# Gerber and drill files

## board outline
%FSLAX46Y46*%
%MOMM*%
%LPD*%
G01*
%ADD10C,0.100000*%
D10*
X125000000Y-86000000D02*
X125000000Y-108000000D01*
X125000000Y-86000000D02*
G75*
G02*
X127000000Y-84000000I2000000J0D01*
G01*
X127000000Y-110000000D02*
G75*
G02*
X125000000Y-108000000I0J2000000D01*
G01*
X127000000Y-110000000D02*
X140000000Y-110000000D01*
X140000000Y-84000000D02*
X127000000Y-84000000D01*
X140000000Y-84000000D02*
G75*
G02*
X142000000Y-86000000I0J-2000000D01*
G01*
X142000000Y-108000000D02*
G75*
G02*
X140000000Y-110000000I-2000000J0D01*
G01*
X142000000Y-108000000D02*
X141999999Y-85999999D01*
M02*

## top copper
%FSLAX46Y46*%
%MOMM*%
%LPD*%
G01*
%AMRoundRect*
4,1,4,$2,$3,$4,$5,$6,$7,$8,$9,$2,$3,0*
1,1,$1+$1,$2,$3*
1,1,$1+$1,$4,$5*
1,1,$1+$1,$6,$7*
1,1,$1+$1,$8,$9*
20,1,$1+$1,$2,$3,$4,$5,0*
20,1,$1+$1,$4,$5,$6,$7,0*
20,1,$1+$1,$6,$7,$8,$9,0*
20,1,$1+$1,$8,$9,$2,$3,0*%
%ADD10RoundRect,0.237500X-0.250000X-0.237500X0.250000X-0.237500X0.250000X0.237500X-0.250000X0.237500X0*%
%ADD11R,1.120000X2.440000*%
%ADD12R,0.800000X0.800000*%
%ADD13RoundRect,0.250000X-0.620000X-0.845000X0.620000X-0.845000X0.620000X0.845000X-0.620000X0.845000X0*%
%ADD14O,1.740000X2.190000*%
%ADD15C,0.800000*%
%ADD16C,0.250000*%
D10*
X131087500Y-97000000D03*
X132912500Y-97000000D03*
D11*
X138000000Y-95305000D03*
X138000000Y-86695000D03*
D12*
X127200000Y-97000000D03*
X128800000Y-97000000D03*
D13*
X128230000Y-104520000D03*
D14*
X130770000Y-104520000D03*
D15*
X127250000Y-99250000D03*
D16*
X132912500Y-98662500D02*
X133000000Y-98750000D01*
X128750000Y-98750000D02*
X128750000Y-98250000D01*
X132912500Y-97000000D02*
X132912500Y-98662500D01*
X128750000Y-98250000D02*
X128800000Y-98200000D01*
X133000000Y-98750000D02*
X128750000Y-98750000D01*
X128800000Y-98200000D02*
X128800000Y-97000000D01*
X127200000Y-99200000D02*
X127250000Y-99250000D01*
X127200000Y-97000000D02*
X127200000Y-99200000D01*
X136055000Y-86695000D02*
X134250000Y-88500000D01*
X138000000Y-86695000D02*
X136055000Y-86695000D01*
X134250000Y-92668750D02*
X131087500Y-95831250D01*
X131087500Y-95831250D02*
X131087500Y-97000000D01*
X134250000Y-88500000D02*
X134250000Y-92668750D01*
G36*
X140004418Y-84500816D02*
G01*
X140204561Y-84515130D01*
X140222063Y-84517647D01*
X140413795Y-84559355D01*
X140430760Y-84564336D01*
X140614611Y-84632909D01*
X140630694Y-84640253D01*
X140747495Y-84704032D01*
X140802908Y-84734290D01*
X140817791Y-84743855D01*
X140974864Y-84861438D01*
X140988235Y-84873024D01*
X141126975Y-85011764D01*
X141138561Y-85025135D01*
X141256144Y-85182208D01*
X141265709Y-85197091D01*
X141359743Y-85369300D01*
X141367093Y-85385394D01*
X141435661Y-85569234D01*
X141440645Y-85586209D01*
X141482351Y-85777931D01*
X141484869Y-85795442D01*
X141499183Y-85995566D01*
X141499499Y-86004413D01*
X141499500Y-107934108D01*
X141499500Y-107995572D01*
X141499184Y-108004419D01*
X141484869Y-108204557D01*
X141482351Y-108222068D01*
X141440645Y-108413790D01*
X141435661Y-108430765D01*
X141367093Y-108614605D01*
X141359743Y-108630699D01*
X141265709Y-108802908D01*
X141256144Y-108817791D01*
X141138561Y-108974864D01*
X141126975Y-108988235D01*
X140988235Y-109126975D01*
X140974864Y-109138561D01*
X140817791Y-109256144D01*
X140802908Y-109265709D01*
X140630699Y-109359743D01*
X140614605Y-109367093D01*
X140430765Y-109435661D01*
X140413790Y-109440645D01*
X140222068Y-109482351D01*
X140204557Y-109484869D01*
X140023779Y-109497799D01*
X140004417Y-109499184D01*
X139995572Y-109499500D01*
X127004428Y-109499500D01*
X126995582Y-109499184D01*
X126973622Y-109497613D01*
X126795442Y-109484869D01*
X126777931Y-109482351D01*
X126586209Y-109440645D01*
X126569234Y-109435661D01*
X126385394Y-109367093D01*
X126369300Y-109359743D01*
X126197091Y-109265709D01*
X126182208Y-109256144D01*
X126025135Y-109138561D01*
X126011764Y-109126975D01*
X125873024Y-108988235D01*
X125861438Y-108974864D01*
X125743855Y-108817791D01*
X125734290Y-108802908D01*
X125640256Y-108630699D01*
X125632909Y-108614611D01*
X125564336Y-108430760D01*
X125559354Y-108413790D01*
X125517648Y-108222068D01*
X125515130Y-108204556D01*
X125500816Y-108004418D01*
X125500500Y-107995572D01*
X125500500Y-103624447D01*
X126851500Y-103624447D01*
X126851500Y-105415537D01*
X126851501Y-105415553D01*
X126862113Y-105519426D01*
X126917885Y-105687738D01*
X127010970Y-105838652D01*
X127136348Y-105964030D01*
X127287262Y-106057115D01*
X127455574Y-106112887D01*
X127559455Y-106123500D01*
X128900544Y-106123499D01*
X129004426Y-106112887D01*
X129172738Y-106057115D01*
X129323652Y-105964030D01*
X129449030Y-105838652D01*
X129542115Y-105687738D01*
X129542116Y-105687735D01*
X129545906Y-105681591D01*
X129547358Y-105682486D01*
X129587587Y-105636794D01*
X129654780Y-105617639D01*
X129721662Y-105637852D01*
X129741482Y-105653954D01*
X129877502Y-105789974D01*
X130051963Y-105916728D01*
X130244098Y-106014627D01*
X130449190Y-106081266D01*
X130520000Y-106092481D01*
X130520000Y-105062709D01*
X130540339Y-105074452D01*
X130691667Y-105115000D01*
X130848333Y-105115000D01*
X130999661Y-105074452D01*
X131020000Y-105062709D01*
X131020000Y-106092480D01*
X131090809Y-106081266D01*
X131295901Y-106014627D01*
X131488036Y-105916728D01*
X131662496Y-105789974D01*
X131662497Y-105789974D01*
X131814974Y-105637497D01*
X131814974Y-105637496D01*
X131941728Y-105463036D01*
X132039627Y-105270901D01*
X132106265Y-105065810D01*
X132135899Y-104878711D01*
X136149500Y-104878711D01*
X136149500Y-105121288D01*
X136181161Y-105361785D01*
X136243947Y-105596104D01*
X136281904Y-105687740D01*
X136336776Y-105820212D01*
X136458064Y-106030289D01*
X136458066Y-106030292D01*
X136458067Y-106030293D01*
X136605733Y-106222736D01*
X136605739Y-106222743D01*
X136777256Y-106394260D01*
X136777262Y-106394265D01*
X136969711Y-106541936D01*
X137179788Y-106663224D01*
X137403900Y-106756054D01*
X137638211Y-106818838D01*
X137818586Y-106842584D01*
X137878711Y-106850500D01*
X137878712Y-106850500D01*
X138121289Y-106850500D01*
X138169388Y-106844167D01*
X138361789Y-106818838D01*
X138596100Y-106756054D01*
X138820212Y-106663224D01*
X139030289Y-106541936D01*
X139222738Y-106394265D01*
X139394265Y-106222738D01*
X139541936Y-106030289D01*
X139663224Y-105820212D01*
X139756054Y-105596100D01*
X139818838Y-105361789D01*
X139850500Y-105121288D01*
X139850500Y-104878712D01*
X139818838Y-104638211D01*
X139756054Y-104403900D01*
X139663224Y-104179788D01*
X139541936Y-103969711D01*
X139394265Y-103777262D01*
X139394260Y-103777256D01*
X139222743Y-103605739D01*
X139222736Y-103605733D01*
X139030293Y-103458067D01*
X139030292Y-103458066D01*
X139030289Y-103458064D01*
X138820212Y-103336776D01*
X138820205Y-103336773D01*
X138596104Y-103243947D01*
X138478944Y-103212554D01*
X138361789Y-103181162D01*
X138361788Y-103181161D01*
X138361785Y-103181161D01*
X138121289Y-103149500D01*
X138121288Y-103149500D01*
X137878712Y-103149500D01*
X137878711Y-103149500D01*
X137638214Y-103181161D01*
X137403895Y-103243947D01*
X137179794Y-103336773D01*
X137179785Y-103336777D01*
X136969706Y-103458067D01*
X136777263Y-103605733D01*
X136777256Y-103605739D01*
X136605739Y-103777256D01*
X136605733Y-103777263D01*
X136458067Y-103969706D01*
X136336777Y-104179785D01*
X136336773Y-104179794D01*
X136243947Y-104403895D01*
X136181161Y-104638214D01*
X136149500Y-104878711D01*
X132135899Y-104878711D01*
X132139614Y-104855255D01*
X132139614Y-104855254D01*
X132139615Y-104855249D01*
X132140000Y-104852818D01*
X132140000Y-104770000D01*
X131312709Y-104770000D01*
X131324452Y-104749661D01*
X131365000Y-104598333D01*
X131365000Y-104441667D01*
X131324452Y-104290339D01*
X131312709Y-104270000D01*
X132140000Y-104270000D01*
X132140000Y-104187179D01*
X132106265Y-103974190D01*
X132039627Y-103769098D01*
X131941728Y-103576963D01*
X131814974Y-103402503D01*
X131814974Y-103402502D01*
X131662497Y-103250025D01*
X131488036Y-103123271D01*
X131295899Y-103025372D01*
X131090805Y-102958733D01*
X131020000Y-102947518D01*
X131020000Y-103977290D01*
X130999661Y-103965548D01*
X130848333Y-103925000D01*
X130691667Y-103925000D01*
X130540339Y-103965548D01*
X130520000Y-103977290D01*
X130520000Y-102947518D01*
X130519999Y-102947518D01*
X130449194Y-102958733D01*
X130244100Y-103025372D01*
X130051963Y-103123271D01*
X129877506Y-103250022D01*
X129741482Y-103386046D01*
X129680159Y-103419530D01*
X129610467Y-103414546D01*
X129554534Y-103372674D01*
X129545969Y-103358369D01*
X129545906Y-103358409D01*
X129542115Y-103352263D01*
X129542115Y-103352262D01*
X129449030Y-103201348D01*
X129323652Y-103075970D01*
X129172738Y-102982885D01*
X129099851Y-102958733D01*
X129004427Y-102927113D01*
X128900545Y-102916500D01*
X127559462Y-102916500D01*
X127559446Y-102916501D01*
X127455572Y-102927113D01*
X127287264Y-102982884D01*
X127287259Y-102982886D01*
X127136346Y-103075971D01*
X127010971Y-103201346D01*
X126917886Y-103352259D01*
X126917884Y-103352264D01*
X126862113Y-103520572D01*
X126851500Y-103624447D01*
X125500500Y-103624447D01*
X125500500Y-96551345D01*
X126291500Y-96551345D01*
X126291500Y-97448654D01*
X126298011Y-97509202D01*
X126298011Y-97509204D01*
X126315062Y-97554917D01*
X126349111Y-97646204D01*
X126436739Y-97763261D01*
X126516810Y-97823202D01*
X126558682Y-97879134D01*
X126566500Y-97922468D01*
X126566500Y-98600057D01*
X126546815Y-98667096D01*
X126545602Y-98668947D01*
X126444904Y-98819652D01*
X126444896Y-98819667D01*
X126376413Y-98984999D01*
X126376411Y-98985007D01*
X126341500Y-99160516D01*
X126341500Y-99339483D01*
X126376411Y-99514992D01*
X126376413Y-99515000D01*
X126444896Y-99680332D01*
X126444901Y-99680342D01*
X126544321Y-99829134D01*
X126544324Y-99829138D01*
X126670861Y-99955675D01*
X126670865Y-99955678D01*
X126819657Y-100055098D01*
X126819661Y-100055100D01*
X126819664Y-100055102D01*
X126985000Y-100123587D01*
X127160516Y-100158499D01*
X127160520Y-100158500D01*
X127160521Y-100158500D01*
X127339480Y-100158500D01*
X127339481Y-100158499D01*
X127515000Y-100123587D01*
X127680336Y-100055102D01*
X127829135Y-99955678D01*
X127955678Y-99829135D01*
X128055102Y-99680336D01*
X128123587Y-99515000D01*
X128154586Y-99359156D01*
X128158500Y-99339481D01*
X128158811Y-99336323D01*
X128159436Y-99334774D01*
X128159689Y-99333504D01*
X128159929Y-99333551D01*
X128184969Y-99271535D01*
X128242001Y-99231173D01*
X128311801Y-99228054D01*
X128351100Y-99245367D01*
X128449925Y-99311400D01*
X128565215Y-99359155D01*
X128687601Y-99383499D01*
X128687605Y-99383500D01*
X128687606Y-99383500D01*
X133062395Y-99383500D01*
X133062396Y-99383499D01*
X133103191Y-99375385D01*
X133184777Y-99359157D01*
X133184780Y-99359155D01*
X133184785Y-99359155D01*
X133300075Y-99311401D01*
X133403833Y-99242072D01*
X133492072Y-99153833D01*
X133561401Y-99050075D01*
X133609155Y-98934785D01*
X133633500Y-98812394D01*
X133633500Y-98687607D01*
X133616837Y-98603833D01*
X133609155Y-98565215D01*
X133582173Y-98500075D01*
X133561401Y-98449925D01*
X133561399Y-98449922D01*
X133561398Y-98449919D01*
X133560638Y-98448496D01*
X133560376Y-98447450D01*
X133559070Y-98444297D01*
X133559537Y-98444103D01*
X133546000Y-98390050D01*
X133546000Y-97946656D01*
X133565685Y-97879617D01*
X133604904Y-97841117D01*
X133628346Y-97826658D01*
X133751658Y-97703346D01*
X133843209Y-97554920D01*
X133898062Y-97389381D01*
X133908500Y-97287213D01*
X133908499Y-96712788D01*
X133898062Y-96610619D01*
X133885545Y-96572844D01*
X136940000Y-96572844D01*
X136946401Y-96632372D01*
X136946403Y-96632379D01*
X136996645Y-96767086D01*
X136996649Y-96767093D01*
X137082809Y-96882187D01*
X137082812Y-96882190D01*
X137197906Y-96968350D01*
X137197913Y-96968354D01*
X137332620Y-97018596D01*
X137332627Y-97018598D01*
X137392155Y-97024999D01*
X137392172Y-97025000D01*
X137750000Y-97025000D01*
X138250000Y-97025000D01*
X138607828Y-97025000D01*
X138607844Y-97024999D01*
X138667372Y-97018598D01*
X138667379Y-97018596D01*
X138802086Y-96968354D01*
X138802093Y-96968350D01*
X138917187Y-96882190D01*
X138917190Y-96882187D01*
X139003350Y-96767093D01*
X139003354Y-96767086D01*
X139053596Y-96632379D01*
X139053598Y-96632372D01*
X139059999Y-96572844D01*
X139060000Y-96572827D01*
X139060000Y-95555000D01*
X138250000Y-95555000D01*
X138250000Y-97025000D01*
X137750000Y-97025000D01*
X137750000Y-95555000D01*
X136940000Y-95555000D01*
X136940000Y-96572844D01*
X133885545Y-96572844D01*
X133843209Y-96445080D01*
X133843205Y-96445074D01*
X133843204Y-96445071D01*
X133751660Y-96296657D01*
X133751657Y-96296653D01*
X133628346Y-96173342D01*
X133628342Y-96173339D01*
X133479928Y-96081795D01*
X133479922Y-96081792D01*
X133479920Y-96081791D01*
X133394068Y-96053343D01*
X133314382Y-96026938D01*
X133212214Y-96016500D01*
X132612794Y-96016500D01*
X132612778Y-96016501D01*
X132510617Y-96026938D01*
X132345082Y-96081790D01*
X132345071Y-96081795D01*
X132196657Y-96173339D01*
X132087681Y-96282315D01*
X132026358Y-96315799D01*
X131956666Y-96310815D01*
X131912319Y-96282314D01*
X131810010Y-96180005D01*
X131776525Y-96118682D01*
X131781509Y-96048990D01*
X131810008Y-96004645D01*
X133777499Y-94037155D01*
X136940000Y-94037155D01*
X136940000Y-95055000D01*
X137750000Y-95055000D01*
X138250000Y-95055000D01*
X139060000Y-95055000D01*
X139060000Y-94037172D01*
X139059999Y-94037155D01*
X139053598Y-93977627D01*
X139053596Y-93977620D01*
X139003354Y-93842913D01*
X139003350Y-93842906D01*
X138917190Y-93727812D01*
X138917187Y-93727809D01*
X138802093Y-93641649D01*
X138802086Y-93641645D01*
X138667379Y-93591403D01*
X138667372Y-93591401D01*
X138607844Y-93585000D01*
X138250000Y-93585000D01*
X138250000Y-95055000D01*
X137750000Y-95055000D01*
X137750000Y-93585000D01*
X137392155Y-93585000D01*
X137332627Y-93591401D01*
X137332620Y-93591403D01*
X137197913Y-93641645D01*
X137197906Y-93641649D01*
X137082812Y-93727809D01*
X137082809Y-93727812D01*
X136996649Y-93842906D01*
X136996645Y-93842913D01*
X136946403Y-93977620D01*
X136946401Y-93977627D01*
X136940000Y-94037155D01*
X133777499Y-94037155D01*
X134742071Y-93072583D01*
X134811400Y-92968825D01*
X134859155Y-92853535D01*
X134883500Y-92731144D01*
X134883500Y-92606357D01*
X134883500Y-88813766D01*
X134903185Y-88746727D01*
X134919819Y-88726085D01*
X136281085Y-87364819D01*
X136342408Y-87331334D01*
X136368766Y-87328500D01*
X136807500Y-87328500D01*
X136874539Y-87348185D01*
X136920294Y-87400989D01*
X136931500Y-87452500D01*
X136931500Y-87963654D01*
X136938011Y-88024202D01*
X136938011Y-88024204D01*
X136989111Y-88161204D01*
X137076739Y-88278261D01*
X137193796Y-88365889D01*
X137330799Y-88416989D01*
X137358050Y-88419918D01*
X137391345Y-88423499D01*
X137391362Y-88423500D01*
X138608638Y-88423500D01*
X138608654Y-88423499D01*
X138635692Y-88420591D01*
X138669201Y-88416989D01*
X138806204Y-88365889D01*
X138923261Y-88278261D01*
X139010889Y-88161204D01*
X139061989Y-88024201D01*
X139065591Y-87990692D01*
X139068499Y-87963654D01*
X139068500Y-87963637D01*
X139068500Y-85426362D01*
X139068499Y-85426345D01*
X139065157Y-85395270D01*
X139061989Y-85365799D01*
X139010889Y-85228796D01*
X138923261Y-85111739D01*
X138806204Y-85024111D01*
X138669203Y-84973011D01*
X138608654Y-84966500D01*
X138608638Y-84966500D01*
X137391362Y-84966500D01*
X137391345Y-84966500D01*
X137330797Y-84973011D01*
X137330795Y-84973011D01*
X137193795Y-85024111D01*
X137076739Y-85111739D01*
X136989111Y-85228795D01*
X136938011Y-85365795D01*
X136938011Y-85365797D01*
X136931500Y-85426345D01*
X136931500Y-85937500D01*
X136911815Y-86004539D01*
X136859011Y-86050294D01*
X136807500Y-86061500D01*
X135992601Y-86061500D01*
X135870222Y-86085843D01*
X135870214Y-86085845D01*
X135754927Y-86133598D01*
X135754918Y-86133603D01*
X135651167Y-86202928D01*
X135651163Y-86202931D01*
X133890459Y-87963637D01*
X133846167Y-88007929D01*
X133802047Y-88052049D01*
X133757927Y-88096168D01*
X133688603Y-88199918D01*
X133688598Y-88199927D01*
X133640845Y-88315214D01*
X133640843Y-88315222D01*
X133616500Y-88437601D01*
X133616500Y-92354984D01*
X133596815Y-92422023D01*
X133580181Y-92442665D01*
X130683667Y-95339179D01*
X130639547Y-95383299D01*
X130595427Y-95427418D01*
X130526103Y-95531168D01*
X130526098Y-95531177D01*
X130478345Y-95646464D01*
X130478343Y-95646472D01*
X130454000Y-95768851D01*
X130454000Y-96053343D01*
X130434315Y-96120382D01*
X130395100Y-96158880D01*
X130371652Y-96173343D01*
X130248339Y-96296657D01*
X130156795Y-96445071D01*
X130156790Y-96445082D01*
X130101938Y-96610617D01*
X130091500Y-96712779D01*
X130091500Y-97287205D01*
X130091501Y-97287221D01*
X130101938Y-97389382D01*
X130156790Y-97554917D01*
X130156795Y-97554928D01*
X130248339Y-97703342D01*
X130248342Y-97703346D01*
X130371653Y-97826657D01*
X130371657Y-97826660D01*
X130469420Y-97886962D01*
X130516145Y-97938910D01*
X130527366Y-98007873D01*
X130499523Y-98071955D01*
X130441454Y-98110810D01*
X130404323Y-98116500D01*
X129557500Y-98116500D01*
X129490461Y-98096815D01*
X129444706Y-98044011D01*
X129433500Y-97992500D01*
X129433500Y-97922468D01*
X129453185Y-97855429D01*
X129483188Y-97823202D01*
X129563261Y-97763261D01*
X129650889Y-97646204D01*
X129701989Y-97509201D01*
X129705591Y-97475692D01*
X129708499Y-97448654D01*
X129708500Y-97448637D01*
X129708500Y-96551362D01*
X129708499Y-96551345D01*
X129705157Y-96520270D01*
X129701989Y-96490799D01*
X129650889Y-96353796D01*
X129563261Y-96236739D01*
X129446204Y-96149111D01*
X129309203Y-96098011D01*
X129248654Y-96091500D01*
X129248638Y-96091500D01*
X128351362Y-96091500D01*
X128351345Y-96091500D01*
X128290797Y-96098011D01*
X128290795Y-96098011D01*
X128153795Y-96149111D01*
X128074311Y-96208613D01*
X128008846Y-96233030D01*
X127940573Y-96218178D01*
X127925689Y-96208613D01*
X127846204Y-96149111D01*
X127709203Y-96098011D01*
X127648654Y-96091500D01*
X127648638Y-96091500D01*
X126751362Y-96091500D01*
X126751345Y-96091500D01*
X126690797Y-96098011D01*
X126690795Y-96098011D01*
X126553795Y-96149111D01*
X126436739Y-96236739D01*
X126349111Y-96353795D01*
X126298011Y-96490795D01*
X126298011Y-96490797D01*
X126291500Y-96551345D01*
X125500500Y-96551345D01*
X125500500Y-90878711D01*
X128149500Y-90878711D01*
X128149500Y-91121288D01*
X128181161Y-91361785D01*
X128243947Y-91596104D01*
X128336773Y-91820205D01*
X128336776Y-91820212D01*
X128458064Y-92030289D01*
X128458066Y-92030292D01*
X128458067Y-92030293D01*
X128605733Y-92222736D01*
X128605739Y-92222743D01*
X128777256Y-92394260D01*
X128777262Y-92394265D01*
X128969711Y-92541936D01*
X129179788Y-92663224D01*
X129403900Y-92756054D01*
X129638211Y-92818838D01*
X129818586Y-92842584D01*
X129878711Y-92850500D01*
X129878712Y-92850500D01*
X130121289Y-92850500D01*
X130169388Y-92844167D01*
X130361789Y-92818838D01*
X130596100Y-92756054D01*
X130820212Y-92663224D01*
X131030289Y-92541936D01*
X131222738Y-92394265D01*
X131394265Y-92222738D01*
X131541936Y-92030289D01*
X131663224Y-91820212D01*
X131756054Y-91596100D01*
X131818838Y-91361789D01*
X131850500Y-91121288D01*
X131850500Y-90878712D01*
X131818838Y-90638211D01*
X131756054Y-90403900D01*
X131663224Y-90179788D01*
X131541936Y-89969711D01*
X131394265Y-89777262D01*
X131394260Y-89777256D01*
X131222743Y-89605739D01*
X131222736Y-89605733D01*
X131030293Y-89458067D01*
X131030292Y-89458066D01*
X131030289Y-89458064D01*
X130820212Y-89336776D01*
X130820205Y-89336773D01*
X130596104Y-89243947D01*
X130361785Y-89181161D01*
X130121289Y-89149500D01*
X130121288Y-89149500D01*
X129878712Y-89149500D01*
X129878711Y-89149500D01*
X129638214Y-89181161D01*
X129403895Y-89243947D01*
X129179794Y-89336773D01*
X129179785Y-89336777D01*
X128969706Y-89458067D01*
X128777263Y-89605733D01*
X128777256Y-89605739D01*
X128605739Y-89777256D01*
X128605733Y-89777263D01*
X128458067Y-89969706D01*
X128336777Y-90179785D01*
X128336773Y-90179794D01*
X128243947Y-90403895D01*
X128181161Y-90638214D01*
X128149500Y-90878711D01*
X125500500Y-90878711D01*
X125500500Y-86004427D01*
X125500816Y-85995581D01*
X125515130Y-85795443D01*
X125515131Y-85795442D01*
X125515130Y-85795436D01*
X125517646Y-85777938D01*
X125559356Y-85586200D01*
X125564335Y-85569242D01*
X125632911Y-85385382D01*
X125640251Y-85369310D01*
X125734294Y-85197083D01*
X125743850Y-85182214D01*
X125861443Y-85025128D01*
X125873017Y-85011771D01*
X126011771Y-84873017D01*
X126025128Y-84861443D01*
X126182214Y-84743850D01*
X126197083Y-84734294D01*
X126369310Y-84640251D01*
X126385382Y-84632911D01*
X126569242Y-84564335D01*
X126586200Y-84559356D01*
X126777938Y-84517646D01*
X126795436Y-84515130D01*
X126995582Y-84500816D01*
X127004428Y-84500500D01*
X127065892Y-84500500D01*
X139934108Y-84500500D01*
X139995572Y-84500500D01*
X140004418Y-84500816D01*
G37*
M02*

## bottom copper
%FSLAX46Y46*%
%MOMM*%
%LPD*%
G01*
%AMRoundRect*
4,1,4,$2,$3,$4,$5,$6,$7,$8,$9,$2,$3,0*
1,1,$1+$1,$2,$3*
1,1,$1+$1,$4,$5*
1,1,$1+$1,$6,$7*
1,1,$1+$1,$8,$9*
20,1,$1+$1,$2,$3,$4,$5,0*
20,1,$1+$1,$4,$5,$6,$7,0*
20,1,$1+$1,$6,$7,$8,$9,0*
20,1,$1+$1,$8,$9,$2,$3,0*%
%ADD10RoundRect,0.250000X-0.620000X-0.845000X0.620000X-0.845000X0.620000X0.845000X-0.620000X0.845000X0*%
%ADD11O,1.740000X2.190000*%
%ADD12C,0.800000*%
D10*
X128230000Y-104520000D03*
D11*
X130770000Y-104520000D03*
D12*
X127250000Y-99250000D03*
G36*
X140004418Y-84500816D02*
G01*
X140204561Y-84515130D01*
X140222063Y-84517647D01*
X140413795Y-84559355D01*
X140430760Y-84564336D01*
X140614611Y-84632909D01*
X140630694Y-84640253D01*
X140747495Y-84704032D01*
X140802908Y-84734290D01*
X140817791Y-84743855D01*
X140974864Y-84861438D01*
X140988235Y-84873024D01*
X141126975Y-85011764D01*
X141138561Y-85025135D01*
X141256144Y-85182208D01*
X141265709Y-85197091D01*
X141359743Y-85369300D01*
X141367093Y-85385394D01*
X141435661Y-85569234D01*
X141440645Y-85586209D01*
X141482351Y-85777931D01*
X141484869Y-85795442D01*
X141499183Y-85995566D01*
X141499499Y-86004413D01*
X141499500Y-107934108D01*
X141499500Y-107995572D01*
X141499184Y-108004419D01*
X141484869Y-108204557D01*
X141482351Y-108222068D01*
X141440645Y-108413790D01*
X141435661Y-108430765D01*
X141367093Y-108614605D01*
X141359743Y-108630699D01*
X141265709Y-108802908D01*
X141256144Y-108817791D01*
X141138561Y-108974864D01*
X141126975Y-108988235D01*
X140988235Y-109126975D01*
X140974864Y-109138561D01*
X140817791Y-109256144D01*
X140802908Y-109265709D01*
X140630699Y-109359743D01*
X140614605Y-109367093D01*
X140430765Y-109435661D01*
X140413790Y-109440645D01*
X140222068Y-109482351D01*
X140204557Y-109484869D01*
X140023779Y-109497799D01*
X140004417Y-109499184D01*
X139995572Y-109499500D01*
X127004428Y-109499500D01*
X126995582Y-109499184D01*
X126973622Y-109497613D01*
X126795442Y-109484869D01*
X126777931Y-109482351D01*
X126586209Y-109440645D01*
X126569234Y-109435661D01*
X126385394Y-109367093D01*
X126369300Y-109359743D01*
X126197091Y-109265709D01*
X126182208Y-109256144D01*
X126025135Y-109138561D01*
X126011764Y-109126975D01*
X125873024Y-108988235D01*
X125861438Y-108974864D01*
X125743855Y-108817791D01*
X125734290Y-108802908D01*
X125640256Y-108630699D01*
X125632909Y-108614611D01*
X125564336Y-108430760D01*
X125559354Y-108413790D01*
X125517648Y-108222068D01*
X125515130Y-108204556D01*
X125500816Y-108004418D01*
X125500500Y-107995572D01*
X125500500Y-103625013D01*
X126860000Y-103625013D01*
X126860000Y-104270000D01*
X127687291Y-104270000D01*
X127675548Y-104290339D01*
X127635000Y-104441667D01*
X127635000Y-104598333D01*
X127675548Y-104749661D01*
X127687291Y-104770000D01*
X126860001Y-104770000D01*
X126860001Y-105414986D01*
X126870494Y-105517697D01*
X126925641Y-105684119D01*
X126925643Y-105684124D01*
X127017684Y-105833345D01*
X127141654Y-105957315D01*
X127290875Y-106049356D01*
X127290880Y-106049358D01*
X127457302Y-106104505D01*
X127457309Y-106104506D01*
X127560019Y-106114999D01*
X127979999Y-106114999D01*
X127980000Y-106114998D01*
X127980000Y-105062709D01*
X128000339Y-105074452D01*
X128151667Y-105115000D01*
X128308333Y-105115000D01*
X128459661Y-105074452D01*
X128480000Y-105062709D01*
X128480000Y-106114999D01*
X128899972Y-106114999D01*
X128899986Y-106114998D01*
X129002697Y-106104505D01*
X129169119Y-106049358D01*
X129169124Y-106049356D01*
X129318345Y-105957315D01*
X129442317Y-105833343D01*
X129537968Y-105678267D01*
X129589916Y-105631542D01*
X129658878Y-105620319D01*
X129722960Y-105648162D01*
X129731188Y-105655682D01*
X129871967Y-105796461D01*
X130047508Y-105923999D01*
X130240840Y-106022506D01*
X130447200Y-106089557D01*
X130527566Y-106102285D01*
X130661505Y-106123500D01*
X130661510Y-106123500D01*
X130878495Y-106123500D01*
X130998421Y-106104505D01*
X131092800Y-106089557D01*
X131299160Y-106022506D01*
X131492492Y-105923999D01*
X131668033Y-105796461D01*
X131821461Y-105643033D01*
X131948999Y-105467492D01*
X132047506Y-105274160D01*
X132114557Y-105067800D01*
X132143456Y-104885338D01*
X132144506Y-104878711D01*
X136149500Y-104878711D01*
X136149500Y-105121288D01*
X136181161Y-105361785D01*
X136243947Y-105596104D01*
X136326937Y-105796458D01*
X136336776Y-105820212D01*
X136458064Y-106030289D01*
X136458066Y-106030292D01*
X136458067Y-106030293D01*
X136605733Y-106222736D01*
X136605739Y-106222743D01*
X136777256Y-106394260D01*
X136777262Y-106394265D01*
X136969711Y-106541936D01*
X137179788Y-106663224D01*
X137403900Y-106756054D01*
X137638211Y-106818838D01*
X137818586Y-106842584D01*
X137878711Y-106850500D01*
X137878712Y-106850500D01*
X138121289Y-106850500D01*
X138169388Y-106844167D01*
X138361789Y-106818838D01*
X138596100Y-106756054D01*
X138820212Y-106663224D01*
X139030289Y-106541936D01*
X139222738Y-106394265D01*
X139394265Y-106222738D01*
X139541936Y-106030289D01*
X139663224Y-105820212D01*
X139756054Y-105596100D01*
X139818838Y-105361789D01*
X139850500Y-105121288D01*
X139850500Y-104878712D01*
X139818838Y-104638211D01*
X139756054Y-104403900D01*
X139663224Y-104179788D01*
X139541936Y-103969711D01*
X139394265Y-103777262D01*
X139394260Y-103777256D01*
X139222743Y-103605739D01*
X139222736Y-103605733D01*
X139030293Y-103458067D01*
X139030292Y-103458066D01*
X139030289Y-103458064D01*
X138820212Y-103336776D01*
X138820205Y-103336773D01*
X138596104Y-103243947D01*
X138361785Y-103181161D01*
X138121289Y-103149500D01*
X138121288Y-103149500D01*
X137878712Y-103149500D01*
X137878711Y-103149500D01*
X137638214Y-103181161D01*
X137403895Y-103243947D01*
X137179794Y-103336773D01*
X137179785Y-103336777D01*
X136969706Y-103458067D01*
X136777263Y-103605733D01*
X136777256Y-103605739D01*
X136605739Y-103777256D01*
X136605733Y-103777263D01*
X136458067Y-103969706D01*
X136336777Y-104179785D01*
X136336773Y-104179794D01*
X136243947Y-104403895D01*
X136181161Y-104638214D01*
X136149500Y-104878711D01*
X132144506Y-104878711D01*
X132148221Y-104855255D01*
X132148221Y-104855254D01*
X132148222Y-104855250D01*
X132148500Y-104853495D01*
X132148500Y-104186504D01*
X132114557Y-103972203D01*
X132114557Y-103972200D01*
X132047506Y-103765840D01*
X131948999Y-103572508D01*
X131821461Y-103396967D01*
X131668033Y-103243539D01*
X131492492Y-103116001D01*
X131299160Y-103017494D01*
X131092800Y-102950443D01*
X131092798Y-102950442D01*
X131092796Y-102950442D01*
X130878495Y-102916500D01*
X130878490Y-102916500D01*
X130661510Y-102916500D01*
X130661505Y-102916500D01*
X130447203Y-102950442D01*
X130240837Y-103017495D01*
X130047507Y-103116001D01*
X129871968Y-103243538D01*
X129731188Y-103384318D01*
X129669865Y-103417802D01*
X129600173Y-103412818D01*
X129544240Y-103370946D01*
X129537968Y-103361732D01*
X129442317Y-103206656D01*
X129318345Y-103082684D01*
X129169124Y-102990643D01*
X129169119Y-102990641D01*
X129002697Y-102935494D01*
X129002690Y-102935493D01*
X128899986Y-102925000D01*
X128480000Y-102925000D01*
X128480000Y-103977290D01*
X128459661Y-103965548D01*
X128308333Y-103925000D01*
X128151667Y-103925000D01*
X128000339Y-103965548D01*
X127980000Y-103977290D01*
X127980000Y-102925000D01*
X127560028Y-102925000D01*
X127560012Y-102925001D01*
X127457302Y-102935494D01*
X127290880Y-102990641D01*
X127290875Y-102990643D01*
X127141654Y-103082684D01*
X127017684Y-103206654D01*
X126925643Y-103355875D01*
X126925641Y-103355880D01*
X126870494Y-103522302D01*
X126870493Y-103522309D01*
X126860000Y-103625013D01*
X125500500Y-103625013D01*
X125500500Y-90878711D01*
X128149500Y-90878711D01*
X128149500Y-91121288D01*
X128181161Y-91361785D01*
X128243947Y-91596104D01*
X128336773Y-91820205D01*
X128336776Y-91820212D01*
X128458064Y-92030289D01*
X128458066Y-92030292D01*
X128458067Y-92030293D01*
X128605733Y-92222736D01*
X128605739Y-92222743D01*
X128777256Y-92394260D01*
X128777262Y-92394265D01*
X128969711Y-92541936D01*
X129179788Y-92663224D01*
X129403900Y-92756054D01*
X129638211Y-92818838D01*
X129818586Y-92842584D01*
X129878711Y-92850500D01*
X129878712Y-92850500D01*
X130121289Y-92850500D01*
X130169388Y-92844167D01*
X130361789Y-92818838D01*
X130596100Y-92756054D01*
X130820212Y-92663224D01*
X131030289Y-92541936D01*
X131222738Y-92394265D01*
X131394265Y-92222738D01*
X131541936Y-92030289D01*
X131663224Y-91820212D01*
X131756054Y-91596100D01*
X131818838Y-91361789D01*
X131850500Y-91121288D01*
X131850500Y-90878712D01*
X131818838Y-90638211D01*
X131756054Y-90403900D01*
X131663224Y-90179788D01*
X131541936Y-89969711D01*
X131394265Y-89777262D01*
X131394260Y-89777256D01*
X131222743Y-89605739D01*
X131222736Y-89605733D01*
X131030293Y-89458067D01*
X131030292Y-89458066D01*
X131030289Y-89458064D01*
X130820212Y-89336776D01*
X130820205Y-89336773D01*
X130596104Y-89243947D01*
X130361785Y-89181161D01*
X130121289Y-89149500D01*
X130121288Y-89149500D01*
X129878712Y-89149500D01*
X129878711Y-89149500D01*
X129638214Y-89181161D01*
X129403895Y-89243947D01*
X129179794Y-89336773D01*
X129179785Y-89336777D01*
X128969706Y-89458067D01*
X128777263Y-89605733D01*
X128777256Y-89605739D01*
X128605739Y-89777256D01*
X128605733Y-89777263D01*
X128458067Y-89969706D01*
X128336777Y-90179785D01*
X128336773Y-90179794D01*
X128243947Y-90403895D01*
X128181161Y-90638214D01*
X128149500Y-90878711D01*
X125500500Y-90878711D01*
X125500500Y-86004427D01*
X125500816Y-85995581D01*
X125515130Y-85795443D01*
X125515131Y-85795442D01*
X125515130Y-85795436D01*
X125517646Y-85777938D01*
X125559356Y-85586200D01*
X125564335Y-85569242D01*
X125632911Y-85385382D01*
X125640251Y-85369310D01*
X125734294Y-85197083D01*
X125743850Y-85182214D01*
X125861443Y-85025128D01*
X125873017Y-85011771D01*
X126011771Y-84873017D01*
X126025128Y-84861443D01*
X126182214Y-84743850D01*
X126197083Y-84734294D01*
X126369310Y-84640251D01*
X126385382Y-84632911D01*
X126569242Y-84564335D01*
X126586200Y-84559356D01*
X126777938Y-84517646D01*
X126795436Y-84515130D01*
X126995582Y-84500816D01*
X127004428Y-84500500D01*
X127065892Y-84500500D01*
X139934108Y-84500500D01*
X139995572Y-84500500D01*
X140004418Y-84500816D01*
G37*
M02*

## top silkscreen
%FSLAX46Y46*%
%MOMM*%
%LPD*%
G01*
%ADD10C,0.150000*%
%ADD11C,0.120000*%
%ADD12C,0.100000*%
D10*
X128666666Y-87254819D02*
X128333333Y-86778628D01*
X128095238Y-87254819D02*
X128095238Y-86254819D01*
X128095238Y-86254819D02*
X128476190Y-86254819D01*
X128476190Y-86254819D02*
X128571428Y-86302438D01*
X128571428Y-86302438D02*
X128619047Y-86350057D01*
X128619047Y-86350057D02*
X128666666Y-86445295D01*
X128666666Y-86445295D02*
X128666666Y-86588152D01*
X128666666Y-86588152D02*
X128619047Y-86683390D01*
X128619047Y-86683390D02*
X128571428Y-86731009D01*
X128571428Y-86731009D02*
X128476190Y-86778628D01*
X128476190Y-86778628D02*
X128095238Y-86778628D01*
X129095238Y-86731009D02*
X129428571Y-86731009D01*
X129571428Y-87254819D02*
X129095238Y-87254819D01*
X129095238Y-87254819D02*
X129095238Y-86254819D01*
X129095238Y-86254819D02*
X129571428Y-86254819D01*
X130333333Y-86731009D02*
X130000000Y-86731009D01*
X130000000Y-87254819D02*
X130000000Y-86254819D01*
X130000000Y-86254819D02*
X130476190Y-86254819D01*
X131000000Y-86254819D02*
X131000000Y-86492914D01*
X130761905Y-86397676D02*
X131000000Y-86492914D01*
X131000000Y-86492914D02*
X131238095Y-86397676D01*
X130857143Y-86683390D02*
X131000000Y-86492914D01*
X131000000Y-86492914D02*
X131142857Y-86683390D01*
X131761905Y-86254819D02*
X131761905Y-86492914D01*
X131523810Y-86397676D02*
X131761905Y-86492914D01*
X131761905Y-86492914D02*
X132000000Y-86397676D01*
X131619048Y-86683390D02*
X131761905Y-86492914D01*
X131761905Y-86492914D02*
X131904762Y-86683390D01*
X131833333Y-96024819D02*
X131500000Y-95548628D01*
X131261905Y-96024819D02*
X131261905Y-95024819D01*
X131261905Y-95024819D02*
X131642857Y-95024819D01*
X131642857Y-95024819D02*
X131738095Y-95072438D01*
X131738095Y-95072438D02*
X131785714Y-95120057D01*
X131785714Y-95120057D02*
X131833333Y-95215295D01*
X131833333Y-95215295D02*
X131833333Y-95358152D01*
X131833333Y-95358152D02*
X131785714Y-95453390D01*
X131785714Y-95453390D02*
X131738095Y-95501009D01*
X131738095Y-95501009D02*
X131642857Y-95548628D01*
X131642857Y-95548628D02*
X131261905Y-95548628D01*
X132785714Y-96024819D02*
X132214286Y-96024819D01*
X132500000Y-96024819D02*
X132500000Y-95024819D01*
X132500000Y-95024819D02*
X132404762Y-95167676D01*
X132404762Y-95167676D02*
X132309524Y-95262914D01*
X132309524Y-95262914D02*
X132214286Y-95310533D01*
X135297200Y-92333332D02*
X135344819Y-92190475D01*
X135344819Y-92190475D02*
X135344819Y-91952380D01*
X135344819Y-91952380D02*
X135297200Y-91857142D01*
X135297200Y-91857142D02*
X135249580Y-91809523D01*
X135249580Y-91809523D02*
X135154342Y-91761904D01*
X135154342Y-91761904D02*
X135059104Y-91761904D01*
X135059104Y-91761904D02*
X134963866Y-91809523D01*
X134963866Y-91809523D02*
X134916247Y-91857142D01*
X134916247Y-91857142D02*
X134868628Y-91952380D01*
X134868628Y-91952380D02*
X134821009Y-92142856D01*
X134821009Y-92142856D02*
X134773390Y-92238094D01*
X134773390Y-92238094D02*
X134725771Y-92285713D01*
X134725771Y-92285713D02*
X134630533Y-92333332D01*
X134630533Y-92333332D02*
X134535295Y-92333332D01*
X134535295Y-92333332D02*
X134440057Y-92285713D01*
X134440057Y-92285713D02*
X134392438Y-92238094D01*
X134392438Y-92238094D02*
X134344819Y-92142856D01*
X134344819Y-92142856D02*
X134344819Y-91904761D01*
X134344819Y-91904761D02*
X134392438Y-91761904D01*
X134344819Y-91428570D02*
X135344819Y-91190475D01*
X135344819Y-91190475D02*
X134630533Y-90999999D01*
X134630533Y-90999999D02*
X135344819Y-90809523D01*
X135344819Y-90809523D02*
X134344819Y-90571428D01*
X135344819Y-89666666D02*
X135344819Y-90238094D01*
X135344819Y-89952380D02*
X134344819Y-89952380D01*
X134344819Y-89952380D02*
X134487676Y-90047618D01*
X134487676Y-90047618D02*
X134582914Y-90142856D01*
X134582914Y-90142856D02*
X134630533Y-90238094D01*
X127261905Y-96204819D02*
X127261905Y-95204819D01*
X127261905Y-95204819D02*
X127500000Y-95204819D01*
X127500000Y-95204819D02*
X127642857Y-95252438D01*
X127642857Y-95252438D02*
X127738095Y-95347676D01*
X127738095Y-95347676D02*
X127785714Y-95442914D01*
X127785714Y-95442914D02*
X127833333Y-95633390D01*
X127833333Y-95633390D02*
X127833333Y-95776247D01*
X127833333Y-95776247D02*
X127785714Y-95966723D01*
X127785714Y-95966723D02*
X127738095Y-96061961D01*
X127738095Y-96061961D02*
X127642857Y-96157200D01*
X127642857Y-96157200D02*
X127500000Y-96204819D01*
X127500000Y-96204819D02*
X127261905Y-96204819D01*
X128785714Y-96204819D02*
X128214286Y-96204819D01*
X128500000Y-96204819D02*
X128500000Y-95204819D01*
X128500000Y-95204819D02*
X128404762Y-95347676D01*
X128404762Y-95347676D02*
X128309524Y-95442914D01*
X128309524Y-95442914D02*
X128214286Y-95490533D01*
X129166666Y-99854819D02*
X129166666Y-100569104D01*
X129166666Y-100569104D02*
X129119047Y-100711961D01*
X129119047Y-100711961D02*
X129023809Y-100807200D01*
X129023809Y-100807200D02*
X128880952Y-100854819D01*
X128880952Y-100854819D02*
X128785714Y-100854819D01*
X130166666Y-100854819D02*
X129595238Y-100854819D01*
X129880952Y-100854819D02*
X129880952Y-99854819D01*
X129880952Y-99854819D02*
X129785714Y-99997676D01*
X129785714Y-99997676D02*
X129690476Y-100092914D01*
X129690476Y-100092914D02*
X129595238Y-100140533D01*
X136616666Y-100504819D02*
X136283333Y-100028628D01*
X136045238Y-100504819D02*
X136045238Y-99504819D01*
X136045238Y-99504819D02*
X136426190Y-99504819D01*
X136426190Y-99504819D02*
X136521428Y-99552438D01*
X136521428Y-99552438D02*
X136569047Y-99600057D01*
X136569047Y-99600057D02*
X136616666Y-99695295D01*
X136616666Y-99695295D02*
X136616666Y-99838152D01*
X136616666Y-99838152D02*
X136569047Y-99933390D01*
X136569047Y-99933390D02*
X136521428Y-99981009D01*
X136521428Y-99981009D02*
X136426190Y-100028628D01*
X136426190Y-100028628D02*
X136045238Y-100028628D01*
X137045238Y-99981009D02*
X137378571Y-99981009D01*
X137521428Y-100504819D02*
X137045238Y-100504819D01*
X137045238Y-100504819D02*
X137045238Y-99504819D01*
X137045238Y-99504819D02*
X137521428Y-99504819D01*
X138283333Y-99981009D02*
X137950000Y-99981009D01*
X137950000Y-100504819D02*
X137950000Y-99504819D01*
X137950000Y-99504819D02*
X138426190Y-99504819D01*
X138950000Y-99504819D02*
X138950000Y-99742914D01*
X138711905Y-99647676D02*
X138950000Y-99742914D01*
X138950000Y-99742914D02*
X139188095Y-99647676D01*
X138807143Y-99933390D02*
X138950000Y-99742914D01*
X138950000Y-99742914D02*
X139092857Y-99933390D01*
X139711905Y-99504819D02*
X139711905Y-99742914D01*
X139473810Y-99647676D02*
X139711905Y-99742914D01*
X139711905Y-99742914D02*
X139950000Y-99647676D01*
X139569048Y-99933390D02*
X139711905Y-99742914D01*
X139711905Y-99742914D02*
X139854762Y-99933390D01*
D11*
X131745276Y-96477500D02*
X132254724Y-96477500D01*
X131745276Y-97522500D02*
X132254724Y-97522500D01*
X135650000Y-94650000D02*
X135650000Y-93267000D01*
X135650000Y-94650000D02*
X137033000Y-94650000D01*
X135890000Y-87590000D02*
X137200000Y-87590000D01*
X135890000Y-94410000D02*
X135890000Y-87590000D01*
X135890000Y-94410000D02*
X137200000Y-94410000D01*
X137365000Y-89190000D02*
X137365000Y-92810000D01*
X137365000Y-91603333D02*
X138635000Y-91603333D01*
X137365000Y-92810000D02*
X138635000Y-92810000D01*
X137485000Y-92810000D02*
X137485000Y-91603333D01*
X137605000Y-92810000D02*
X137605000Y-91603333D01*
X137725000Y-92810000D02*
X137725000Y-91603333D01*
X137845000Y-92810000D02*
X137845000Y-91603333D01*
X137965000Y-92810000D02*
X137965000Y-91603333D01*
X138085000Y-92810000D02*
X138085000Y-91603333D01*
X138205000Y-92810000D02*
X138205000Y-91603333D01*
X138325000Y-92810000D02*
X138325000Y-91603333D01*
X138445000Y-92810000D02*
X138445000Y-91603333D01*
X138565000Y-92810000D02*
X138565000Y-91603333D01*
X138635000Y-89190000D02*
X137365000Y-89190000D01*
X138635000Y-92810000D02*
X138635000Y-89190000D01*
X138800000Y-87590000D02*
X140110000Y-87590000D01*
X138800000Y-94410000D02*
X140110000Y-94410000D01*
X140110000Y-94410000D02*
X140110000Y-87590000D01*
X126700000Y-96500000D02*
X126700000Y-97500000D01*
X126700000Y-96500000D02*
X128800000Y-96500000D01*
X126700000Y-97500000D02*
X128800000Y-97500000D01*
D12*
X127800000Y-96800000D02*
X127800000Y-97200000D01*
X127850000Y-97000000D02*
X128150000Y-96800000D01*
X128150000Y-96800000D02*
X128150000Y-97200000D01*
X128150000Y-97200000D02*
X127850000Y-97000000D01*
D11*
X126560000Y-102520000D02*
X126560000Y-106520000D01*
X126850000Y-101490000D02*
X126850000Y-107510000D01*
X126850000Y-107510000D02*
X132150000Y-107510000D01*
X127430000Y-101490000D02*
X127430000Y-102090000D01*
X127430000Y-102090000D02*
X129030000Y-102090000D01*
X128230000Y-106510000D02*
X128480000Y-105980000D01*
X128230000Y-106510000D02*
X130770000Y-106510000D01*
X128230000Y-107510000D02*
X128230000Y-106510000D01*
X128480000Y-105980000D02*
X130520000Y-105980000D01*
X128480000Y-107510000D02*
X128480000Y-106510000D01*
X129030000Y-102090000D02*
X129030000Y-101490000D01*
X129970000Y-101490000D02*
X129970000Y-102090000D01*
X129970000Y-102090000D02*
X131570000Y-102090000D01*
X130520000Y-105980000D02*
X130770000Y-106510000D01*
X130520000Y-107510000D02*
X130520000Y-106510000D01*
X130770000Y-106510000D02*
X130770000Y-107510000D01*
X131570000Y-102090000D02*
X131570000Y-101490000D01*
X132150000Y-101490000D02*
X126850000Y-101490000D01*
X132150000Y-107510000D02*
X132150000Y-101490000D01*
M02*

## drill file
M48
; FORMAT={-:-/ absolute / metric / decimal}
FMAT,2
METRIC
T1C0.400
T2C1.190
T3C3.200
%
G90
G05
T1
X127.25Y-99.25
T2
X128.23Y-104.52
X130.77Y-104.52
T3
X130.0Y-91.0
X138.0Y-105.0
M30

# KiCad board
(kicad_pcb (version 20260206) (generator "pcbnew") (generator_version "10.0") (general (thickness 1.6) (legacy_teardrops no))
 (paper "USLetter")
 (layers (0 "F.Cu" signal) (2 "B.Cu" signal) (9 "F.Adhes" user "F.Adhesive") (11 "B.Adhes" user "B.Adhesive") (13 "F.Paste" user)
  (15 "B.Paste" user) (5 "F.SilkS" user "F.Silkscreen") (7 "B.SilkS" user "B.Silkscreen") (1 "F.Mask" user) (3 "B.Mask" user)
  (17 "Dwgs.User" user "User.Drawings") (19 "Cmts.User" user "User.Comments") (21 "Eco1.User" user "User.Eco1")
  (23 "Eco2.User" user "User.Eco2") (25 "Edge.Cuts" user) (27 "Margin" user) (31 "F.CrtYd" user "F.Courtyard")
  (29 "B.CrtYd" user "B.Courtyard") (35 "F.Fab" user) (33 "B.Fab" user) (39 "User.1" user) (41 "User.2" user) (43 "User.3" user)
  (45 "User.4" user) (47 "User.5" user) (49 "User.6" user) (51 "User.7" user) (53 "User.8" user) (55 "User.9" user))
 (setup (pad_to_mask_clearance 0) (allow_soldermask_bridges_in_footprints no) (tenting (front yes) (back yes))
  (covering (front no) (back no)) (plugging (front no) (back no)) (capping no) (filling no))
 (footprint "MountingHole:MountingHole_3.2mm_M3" (layer "F.Cu") (at 130 91)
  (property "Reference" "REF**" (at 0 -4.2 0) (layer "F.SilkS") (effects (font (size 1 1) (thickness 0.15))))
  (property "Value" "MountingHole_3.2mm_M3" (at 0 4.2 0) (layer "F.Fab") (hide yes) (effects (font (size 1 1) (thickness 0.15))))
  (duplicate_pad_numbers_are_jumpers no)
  (pad "" np_thru_hole circle (at 0 0) (size 3.2 3.2) (drill 3.2) (layers "*.Cu" "*.Mask")))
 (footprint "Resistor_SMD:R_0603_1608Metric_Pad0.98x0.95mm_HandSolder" (layer "F.Cu") (at 132 97)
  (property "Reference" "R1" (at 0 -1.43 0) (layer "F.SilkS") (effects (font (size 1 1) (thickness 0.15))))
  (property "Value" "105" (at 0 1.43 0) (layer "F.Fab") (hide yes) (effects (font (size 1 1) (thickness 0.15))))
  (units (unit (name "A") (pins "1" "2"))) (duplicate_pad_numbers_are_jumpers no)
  (fp_line (start -0.254724 -0.5225) (end 0.254724 -0.5225) (stroke (width 0.12) (type solid)) (layer "F.SilkS"))
  (fp_line (start -0.254724 0.5225) (end 0.254724 0.5225) (stroke (width 0.12) (type solid)) (layer "F.SilkS"))
  (pad "1" smd roundrect (at -0.9125 0) (size 0.975 0.95) (layers "F.Cu" "F.Mask" "F.Paste") (roundrect_rratio 0.25) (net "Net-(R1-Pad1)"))
  (pad "2" smd roundrect (at 0.9125 0) (size 0.975 0.95) (layers "F.Cu" "F.Mask" "F.Paste") (roundrect_rratio 0.25) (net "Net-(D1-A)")))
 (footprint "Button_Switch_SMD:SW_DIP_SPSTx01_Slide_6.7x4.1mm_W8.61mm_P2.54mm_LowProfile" (layer "F.Cu") (at 138 91 90)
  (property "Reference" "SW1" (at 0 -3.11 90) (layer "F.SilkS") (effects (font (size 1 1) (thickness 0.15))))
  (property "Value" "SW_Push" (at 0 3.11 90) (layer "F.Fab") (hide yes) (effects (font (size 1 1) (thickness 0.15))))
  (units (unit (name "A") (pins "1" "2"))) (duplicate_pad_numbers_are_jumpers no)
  (fp_line (start -3.65 -2.35) (end -2.267 -2.35) (stroke (width 0.12) (type solid)) (layer "F.SilkS"))
  (fp_line (start -3.65 -2.35) (end -3.65 -0.967) (stroke (width 0.12) (type solid)) (layer "F.SilkS"))
  (fp_line (start 3.41 -2.11) (end 3.41 -0.8) (stroke (width 0.12) (type solid)) (layer "F.SilkS"))
  (fp_line (start -3.41 -2.11) (end 3.41 -2.11) (stroke (width 0.12) (type solid)) (layer "F.SilkS"))
  (fp_line (start -3.41 -2.11) (end -3.41 -0.8) (stroke (width 0.12) (type solid)) (layer "F.SilkS"))
  (fp_line (start 1.81 -0.635) (end -1.81 -0.635) (stroke (width 0.12) (type solid)) (layer "F.SilkS"))
  (fp_line (start -0.603333 -0.635) (end -0.603333 0.635) (stroke (width 0.12) (type solid)) (layer "F.SilkS"))
  (fp_line (start -1.81 -0.635) (end -1.81 0.635) (stroke (width 0.12) (type solid)) (layer "F.SilkS"))
  (fp_line (start -1.81 -0.515) (end -0.603333 -0.515) (stroke (width 0.12) (type solid)) (layer "F.SilkS"))
  (fp_line (start -1.81 -0.395) (end -0.603333 -0.395) (stroke (width 0.12) (type solid)) (layer "F.SilkS"))
  (fp_line (start -1.81 -0.275) (end -0.603333 -0.275) (stroke (width 0.12) (type solid)) (layer "F.SilkS"))
  (fp_line (start -1.81 -0.155) (end -0.603333 -0.155) (stroke (width 0.12) (type solid)) (layer "F.SilkS"))
  (fp_line (start -1.81 -0.035) (end -0.603333 -0.035) (stroke (width 0.12) (type solid)) (layer "F.SilkS"))
  (fp_line (start -1.81 0.085) (end -0.603333 0.085) (stroke (width 0.12) (type solid)) (layer "F.SilkS"))
  (fp_line (start -1.81 0.205) (end -0.603333 0.205) (stroke (width 0.12) (type solid)) (layer "F.SilkS"))
  (fp_line (start -1.81 0.325) (end -0.603333 0.325) (stroke (width 0.12) (type solid)) (layer "F.SilkS"))
  (fp_line (start -1.81 0.445) (end -0.603333 0.445) (stroke (width 0.12) (type solid)) (layer "F.SilkS"))
  (fp_line (start -1.81 0.565) (end -0.603333 0.565) (stroke (width 0.12) (type solid)) (layer "F.SilkS"))
  (fp_line (start 1.81 0.635) (end 1.81 -0.635) (stroke (width 0.12) (type solid)) (layer "F.SilkS"))
  (fp_line (start -1.81 0.635) (end 1.81 0.635) (stroke (width 0.12) (type solid)) (layer "F.SilkS"))
  (fp_line (start 3.41 0.8) (end 3.41 2.11) (stroke (width 0.12) (type solid)) (layer "F.SilkS"))
  (fp_line (start -3.41 0.8) (end -3.41 2.11) (stroke (width 0.12) (type solid)) (layer "F.SilkS"))
  (fp_line (start -3.41 2.11) (end 3.41 2.11) (stroke (width 0.12) (type solid)) (layer "F.SilkS"))
  (pad "1" smd rect (at -4.305 0 90) (size 2.44 1.12) (layers "F.Cu" "F.Mask" "F.Paste") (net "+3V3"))
  (pad "2" smd rect (at 4.305 0 90) (size 2.44 1.12) (layers "F.Cu" "F.Mask" "F.Paste") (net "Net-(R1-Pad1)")))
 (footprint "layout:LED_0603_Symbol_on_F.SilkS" (layer "F.Cu") (at 128 97)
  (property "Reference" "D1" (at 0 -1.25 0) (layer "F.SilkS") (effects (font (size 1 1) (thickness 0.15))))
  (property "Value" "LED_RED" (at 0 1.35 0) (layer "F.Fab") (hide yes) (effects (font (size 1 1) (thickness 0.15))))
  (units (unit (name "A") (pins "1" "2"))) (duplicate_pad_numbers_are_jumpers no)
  (fp_line (start -1.3 -0.5) (end -1.3 0.5) (stroke (width 0.12) (type solid)) (layer "F.SilkS"))
  (fp_line (start -1.3 -0.5) (end 0.8 -0.5) (stroke (width 0.12) (type solid)) (layer "F.SilkS"))
  (fp_line (start -1.3 0.5) (end 0.8 0.5) (stroke (width 0.12) (type solid)) (layer "F.SilkS"))
  (fp_line (start -0.2 -0.2) (end -0.2 0.2) (stroke (width 0.1) (type solid)) (layer "F.SilkS"))
  (fp_line (start -0.15 0) (end 0.15 -0.2) (stroke (width 0.1) (type solid)) (layer "F.SilkS"))
  (fp_line (start 0.15 -0.2) (end 0.15 0.2) (stroke (width 0.1) (type solid)) (layer "F.SilkS"))
  (fp_line (start 0.15 0.2) (end -0.15 0) (stroke (width 0.1) (type solid)) (layer "F.SilkS"))
  (pad "1" smd rect (at -0.8 0 180) (size 0.8 0.8) (layers "F.Cu" "F.Mask" "F.Paste") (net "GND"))
  (pad "2" smd rect (at 0.8 0 180) (size 0.8 0.8) (layers "F.Cu" "F.Mask" "F.Paste") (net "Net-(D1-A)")))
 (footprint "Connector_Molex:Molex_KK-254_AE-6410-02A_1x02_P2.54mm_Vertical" (layer "F.Cu") (at 128.23 104.52)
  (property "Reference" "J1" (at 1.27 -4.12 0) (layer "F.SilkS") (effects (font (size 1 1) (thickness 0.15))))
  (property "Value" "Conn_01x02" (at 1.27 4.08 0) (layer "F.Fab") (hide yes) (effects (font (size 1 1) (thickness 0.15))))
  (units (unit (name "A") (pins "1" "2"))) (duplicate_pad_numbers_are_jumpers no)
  (fp_line (start -1.67 -2) (end -1.67 2) (stroke (width 0.12) (type solid)) (layer "F.SilkS"))
  (fp_line (start -1.38 -3.03) (end -1.38 2.99) (stroke (width 0.12) (type solid)) (layer "F.SilkS"))
  (fp_line (start -1.38 2.99) (end 3.92 2.99) (stroke (width 0.12) (type solid)) (layer "F.SilkS"))
  (fp_line (start -0.8 -3.03) (end -0.8 -2.43) (stroke (width 0.12) (type solid)) (layer "F.SilkS"))
  (fp_line (start -0.8 -2.43) (end 0.8 -2.43) (stroke (width 0.12) (type solid)) (layer "F.SilkS"))
  (fp_line (start 0 1.99) (end 0.25 1.46) (stroke (width 0.12) (type solid)) (layer "F.SilkS"))
  (fp_line (start 0 1.99) (end 2.54 1.99) (stroke (width 0.12) (type solid)) (layer "F.SilkS"))
  (fp_line (start 0 2.99) (end 0 1.99) (stroke (width 0.12) (type solid)) (layer "F.SilkS"))
  (fp_line (start 0.25 1.46) (end 2.29 1.46) (stroke (width 0.12) (type solid)) (layer "F.SilkS"))
  (fp_line (start 0.25 2.99) (end 0.25 1.99) (stroke (width 0.12) (type solid)) (layer "F.SilkS"))
  (fp_line (start 0.8 -2.43) (end 0.8 -3.03) (stroke (width 0.12) (type solid)) (layer "F.SilkS"))
  (fp_line (start 1.74 -3.03) (end 1.74 -2.43) (stroke (width 0.12) (type solid)) (layer "F.SilkS"))
  (fp_line (start 1.74 -2.43) (end 3.34 -2.43) (stroke (width 0.12) (type solid)) (layer "F.SilkS"))
  (fp_line (start 2.29 1.46) (end 2.54 1.99) (stroke (width 0.12) (type solid)) (layer "F.SilkS"))
  (fp_line (start 2.29 2.99) (end 2.29 1.99) (stroke (width 0.12) (type solid)) (layer "F.SilkS"))
  (fp_line (start 2.54 1.99) (end 2.54 2.99) (stroke (width 0.12) (type solid)) (layer "F.SilkS"))
  (fp_line (start 3.34 -2.43) (end 3.34 -3.03) (stroke (width 0.12) (type solid)) (layer "F.SilkS"))
  (fp_line (start 3.92 -3.03) (end -1.38 -3.03) (stroke (width 0.12) (type solid)) (layer "F.SilkS"))
  (fp_line (start 3.92 2.99) (end 3.92 -3.03) (stroke (width 0.12) (type solid)) (layer "F.SilkS"))
  (pad "1" thru_hole roundrect (at 0 0) (size 1.74 2.19) (drill 1.19) (layers "*.Cu" "*.Mask") (remove_unused_layers no)
   (roundrect_rratio 0.143678) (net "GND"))
  (pad "2" thru_hole oval (at 2.54 0) (size 1.74 2.19) (drill 1.19) (layers "*.Cu" "*.Mask") (remove_unused_layers no) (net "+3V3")))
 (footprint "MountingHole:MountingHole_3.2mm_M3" (layer "F.Cu") (at 138 105)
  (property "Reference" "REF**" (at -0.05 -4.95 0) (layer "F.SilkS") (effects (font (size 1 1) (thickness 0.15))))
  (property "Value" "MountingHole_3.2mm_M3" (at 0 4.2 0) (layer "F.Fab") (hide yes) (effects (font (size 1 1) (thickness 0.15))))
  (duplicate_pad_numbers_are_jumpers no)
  (pad "" np_thru_hole circle (at 0 0) (size 3.2 3.2) (drill 3.2) (layers "*.Cu" "*.Mask")))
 (gr_line (start 125 86) (end 125 108) (stroke (width 0.1) (type default)) (layer "Edge.Cuts"))
 (gr_arc (start 125 86) (mid 125.585786 84.585786) (end 127 84) (stroke (width 0.1) (type default)) (layer "Edge.Cuts"))
 (gr_arc (start 127 110) (mid 125.585786 109.414214) (end 125 108) (stroke (width 0.1) (type default)) (layer "Edge.Cuts"))
 (gr_line (start 127 110) (end 140 110) (stroke (width 0.1) (type default)) (layer "Edge.Cuts"))
 (gr_line (start 140 84) (end 127 84) (stroke (width 0.1) (type default)) (layer "Edge.Cuts"))
 (gr_arc (start 140 84) (mid 141.414214 84.585786) (end 142 86) (stroke (width 0.1) (type default)) (layer "Edge.Cuts"))
 (gr_arc (start 142 108) (mid 141.414214 109.414214) (end 140 110) (stroke (width 0.1) (type default)) (layer "Edge.Cuts"))
 (gr_line (start 142 108) (end 141.999999 85.999999) (stroke (width 0.1) (type default)) (layer "Edge.Cuts"))
 (segment (start 132.9125 98.6625) (end 133 98.75) (width 0.25) (layer "F.Cu") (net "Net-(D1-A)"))
 (segment (start 128.75 98.75) (end 128.75 98.25) (width 0.25) (layer "F.Cu") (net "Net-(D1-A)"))
 (segment (start 132.9125 97) (end 132.9125 98.6625) (width 0.25) (layer "F.Cu") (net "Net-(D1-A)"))
 (segment (start 128.75 98.25) (end 128.8 98.2) (width 0.25) (layer "F.Cu") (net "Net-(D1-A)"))
 (segment (start 133 98.75) (end 128.75 98.75) (width 0.25) (layer "F.Cu") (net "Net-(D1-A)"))
 (segment (start 128.8 98.2) (end 128.8 97) (width 0.25) (layer "F.Cu") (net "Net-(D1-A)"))
 (segment (start 127.2 99.2) (end 127.25 99.25) (width 0.25) (layer "F.Cu") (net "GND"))
 (segment (start 127.2 97) (end 127.2 99.2) (width 0.25) (layer "F.Cu") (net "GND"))
 (via (at 127.25 99.25) (size 0.8) (drill 0.4) (layers "F.Cu" "B.Cu") (free yes) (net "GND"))
 (segment (start 136.055 86.695) (end 134.25 88.5) (width 0.25) (layer "F.Cu") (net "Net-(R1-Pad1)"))
 (segment (start 138 86.695) (end 136.055 86.695) (width 0.25) (layer "F.Cu") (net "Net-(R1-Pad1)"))
 (segment (start 134.25 92.66875) (end 131.0875 95.83125) (width 0.25) (layer "F.Cu") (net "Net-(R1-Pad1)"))
 (segment (start 131.0875 95.83125) (end 131.0875 97) (width 0.25) (layer "F.Cu") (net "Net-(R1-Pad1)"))
 (segment (start 134.25 88.5) (end 134.25 92.66875) (width 0.25) (layer "F.Cu") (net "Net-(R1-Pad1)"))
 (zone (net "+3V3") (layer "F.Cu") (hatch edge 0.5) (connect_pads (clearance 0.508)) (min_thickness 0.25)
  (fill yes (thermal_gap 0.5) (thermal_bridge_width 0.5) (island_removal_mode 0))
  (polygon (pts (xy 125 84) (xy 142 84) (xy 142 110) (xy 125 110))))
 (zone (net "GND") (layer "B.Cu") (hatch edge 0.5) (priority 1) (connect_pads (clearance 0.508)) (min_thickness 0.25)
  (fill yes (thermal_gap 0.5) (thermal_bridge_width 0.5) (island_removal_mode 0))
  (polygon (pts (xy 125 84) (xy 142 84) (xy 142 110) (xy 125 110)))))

